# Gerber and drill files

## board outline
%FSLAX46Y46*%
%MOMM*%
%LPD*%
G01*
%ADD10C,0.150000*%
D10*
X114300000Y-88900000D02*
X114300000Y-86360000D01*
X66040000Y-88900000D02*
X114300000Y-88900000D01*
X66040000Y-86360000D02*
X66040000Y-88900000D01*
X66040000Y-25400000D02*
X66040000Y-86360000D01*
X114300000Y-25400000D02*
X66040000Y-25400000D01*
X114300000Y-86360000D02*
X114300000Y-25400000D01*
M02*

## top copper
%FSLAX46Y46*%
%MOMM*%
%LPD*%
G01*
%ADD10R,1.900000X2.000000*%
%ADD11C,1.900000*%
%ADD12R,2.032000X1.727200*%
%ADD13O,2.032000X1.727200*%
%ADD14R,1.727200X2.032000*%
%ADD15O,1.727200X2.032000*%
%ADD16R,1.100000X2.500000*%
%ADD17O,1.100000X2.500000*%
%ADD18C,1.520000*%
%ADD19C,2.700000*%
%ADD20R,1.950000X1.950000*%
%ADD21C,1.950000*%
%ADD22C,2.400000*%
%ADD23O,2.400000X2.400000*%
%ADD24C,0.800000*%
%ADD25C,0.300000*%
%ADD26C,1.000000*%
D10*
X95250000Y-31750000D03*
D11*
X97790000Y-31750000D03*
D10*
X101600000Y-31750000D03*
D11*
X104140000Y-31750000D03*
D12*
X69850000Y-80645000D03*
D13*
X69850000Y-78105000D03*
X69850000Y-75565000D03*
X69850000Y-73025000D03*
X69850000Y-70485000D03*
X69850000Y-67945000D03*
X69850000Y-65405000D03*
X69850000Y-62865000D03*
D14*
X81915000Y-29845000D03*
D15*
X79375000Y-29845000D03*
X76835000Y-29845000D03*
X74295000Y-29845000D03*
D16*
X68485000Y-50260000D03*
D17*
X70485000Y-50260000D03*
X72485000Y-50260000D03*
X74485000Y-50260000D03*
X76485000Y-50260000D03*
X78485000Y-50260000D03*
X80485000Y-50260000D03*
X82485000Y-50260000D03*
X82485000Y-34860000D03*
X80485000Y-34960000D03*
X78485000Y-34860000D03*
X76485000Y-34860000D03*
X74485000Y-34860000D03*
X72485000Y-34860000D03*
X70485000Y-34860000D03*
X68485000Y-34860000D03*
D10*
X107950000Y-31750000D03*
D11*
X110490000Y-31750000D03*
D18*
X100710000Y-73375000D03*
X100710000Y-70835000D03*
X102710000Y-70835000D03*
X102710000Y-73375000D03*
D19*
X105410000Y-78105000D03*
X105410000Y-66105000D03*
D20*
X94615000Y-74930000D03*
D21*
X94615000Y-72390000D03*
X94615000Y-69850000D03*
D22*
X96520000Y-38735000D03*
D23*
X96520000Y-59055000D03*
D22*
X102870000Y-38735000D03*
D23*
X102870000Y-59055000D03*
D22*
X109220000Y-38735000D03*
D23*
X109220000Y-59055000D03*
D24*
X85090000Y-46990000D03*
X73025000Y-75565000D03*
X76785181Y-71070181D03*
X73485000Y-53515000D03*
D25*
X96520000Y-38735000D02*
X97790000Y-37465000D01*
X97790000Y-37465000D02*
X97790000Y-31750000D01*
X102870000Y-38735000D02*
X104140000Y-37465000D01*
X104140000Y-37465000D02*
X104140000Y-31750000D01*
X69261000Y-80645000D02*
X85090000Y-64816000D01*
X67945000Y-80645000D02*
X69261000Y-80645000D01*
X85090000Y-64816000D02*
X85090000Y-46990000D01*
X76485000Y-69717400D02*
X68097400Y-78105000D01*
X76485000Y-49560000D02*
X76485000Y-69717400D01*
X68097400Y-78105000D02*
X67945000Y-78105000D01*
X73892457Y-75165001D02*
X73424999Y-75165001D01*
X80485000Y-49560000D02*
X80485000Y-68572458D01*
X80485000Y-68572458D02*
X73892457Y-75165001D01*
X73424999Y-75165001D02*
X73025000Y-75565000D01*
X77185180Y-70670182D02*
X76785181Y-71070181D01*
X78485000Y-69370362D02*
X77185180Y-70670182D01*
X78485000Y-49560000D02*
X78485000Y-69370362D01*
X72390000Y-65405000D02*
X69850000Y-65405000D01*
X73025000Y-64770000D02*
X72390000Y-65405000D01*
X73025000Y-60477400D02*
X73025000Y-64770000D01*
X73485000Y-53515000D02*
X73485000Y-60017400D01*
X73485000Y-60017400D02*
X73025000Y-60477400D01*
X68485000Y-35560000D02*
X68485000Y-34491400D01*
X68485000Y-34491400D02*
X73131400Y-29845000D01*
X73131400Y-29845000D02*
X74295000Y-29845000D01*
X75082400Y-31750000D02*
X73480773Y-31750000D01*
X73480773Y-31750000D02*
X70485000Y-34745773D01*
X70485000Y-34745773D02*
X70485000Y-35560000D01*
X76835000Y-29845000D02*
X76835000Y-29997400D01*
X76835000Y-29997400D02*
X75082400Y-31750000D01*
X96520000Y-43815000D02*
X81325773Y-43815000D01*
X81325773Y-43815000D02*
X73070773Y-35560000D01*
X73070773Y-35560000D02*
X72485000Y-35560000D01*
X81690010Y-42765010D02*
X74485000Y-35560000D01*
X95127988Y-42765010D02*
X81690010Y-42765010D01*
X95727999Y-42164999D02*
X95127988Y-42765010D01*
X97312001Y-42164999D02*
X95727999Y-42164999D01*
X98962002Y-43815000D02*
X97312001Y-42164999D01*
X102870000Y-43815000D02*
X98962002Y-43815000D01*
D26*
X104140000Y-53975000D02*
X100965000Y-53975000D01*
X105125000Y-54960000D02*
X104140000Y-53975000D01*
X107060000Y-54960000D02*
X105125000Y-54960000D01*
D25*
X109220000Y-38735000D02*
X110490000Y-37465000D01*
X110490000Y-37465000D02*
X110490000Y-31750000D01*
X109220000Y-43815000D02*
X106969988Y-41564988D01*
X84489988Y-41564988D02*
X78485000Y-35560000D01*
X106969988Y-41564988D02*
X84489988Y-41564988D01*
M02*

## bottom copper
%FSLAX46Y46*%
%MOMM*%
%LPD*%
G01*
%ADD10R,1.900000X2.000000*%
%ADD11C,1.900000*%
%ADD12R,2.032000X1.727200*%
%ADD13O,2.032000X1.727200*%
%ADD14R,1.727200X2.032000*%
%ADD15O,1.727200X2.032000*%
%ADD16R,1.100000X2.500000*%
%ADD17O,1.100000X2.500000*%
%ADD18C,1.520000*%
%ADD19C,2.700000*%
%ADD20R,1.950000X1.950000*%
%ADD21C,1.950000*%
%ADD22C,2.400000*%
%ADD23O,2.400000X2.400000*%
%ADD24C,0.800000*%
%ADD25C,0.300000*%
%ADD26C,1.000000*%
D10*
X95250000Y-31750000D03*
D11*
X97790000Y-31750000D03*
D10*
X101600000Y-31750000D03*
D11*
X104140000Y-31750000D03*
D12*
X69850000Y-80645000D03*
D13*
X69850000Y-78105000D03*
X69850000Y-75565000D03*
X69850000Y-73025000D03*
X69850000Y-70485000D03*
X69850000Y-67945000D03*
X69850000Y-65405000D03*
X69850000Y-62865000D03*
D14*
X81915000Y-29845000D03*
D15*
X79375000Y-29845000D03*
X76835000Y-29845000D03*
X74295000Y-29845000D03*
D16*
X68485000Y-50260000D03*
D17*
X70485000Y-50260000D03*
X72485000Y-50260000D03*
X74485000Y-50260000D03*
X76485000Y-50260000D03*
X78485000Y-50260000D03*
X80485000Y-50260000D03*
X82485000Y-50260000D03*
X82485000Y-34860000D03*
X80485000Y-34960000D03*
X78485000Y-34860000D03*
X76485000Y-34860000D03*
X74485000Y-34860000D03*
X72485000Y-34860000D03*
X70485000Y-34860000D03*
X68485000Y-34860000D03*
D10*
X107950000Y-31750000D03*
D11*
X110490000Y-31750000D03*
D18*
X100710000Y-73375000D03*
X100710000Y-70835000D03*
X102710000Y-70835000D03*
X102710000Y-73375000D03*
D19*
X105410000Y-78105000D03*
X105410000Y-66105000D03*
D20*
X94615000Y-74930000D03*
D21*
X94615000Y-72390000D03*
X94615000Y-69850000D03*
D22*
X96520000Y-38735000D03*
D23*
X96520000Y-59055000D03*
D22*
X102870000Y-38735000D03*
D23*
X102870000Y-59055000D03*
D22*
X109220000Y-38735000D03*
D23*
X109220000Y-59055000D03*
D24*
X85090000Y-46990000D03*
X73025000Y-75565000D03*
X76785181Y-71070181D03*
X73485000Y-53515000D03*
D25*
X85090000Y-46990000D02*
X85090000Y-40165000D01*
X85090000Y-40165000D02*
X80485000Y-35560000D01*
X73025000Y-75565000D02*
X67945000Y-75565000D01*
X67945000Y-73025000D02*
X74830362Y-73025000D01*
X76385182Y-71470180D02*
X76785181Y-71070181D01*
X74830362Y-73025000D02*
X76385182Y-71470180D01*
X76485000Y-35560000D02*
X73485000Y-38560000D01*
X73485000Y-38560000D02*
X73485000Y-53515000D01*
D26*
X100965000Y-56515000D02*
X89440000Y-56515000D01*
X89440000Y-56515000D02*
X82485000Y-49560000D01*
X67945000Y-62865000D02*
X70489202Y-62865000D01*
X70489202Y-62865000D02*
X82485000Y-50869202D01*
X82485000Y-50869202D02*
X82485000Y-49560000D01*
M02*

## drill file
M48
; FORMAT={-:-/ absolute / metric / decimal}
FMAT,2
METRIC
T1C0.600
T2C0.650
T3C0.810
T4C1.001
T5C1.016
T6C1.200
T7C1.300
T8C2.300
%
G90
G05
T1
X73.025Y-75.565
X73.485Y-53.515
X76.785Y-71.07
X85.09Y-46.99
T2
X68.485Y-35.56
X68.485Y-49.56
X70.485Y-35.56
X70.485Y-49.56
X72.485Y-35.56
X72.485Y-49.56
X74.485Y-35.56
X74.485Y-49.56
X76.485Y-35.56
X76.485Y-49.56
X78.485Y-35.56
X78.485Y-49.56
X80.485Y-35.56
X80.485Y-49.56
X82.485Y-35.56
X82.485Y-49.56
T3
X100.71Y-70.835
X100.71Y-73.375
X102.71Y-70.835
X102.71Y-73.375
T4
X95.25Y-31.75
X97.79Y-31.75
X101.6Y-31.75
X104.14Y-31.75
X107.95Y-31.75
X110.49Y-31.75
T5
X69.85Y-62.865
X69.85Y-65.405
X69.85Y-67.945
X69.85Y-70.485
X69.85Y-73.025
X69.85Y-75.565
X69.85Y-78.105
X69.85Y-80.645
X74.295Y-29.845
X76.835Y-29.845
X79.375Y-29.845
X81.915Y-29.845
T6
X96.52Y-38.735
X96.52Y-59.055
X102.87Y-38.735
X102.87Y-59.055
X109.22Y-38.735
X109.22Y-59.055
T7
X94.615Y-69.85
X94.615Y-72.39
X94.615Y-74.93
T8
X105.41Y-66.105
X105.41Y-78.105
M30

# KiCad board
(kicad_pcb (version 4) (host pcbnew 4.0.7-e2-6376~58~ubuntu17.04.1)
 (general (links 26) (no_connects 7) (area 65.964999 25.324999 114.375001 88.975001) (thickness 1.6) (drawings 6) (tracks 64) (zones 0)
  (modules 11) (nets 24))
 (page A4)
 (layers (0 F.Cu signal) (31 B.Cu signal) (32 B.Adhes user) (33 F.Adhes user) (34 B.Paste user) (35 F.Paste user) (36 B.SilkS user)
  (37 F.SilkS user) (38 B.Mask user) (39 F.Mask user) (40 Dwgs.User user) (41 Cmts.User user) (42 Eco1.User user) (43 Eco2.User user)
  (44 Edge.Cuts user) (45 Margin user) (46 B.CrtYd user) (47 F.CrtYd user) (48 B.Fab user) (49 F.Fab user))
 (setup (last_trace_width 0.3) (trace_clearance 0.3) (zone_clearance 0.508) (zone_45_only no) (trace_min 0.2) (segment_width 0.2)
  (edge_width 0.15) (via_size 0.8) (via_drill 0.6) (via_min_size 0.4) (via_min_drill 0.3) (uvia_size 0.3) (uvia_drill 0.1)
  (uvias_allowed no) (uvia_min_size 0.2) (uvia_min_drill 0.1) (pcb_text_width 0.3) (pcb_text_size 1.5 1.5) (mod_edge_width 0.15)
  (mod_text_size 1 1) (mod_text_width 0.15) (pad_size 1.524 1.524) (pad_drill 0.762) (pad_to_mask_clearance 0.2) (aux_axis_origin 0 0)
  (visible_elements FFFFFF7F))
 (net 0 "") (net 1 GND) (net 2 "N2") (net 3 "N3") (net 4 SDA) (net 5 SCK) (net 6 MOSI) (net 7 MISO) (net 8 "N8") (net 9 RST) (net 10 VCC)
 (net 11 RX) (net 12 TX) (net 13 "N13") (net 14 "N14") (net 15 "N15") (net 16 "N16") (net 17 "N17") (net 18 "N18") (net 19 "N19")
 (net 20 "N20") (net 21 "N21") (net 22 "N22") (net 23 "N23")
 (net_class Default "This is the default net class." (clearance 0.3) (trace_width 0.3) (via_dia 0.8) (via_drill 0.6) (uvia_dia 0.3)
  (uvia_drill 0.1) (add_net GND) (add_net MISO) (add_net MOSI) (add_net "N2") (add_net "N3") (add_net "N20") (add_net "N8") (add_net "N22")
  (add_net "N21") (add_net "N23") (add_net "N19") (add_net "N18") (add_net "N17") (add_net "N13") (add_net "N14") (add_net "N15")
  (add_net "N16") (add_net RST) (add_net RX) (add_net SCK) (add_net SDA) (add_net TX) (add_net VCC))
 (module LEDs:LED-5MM (layer F.Cu) (at 95.25 31.75)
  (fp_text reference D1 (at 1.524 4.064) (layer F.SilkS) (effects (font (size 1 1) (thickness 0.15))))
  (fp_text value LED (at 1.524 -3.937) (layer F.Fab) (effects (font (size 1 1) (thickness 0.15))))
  (pad 1 thru_hole rect (at 0 0 90) (size 2 1.9) (drill 1.00076) (layers *.Cu *.Mask) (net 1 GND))
  (pad 2 thru_hole circle (at 2.54 0) (size 1.9 1.9) (drill 1.00076) (layers *.Cu *.Mask) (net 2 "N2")))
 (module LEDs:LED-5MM (layer F.Cu) (at 101.6 31.75)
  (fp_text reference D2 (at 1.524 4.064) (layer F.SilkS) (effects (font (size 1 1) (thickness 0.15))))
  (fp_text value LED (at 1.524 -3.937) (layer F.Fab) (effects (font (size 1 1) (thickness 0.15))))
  (pad 1 thru_hole rect (at 0 0 90) (size 2 1.9) (drill 1.00076) (layers *.Cu *.Mask) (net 1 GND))
  (pad 2 thru_hole circle (at 2.54 0) (size 1.9 1.9) (drill 1.00076) (layers *.Cu *.Mask) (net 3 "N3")))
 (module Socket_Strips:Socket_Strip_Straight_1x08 (layer F.Cu) (at 69.85 80.645 90)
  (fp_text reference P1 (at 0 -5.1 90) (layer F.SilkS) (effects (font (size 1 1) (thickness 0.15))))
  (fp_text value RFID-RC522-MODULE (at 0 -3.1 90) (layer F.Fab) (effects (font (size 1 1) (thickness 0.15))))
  (pad 1 thru_hole rect (at 0 0 90) (size 1.7272 2.032) (drill 1.016) (layers *.Cu *.Mask) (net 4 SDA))
  (pad 2 thru_hole oval (at 2.54 0 90) (size 1.7272 2.032) (drill 1.016) (layers *.Cu *.Mask) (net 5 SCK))
  (pad 3 thru_hole oval (at 5.08 0 90) (size 1.7272 2.032) (drill 1.016) (layers *.Cu *.Mask) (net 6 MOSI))
  (pad 4 thru_hole oval (at 7.62 0 90) (size 1.7272 2.032) (drill 1.016) (layers *.Cu *.Mask) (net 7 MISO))
  (pad 5 thru_hole oval (at 10.16 0 90) (size 1.7272 2.032) (drill 1.016) (layers *.Cu *.Mask) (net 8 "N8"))
  (pad 6 thru_hole oval (at 12.7 0 90) (size 1.7272 2.032) (drill 1.016) (layers *.Cu *.Mask) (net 1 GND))
  (pad 7 thru_hole oval (at 15.24 0 90) (size 1.7272 2.032) (drill 1.016) (layers *.Cu *.Mask) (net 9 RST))
  (pad 8 thru_hole oval (at 17.78 0 90) (size 1.7272 2.032) (drill 1.016) (layers *.Cu *.Mask) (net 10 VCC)))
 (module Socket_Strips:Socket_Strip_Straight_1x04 (layer F.Cu) (at 81.915 29.845 180)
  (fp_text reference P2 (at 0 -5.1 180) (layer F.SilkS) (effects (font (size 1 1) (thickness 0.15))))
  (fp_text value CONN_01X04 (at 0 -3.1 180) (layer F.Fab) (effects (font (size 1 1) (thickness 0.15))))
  (pad 1 thru_hole rect (at 0 0 180) (size 1.7272 2.032) (drill 1.016) (layers *.Cu *.Mask) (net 10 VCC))
  (pad 2 thru_hole oval (at 2.54 0 180) (size 1.7272 2.032) (drill 1.016) (layers *.Cu *.Mask) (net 1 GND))
  (pad 3 thru_hole oval (at 5.08 0 180) (size 1.7272 2.032) (drill 1.016) (layers *.Cu *.Mask) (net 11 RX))
  (pad 4 thru_hole oval (at 7.62 0 180) (size 1.7272 2.032) (drill 1.016) (layers *.Cu *.Mask) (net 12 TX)))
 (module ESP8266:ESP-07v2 (layer F.Cu) (at 68.485 49.56 90)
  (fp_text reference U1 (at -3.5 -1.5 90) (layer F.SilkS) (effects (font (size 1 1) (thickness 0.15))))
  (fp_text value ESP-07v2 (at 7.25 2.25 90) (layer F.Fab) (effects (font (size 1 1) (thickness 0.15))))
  (pad 1 thru_hole rect (at 0 0 90) (size 2.5 1.1) (drill 0.65 (offset -0.7 0)) (layers *.Cu *.Mask F.Paste F.SilkS) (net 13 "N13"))
  (pad 2 thru_hole oval (at 0 2 90) (size 2.5 1.1) (drill 0.65 (offset -0.7 0)) (layers *.Cu *.Mask F.Paste F.SilkS) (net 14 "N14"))
  (pad 3 thru_hole oval (at 0 4 90) (size 2.5 1.1) (drill 0.65 (offset -0.7 0)) (layers *.Cu *.Mask F.Paste F.SilkS) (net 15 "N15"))
  (pad 4 thru_hole oval (at 0 6 90) (size 2.5 1.1) (drill 0.65 (offset -0.7 0)) (layers *.Cu *.Mask F.Paste F.SilkS) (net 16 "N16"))
  (pad 5 thru_hole oval (at 0 8 90) (size 2.5 1.1) (drill 0.65 (offset -0.7 0)) (layers *.Cu *.Mask F.Paste F.SilkS) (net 5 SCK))
  (pad 6 thru_hole oval (at 0 10 90) (size 2.5 1.1) (drill 0.65 (offset -0.7 0)) (layers *.Cu *.Mask F.Paste F.SilkS) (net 7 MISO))
  (pad 7 thru_hole oval (at 0 12 90) (size 2.5 1.1) (drill 0.65 (offset -0.7 0)) (layers *.Cu *.Mask F.Paste F.SilkS) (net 6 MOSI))
  (pad 8 thru_hole oval (at 0 14 90) (size 2.5 1.1) (drill 0.65 (offset -0.7 0)) (layers *.Cu *.Mask F.Paste F.SilkS) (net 10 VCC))
  (pad 9 thru_hole oval (at 14 14 90) (size 2.5 1.1) (drill 0.65 (offset 0.7 0)) (layers *.Cu *.Mask F.Paste F.SilkS) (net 1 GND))
  (pad 10 thru_hole oval (at 14 12 90) (size 2.5 1.1) (drill 0.65 (offset 0.6 0)) (layers *.Cu *.Mask F.Paste F.SilkS) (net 4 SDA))
  (pad 11 thru_hole oval (at 14 10 90) (size 2.5 1.1) (drill 0.65 (offset 0.7 0)) (layers *.Cu *.Mask F.Paste F.SilkS) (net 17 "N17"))
  (pad 12 thru_hole oval (at 14 8 90) (size 2.5 1.1) (drill 0.65 (offset 0.7 0)) (layers *.Cu *.Mask F.Paste F.SilkS) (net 9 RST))
  (pad 13 thru_hole oval (at 14 6 90) (size 2.5 1.1) (drill 0.65 (offset 0.7 0)) (layers *.Cu *.Mask F.Paste F.SilkS) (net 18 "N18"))
  (pad 14 thru_hole oval (at 14 4 90) (size 2.5 1.1) (drill 0.65 (offset 0.7 0)) (layers *.Cu *.Mask F.Paste F.SilkS) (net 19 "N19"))
  (pad 15 thru_hole oval (at 14 2 90) (size 2.5 1.1) (drill 0.65 (offset 0.7 0)) (layers *.Cu *.Mask F.Paste F.SilkS) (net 11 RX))
  (pad 16 thru_hole oval (at 14 0 90) (size 2.5 1.1) (drill 0.65 (offset 0.7 0)) (layers *.Cu *.Mask F.Paste F.SilkS) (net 12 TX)))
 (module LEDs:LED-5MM (layer F.Cu) (at 107.95 31.75)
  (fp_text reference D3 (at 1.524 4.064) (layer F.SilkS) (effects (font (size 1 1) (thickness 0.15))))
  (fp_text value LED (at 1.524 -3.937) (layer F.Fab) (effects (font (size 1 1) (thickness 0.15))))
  (pad 1 thru_hole rect (at 0 0 90) (size 2 1.9) (drill 1.00076) (layers *.Cu *.Mask) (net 1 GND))
  (pad 2 thru_hole circle (at 2.54 0) (size 1.9 1.9) (drill 1.00076) (layers *.Cu *.Mask) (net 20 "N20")))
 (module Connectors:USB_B (layer F.Cu) (at 100.71 70.835)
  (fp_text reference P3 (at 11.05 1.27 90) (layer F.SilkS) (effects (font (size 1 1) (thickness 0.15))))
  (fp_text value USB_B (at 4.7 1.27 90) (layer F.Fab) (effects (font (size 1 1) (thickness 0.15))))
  (pad 2 thru_hole circle (at 0 2.54 270) (size 1.52 1.52) (drill 0.81) (layers *.Cu *.Mask) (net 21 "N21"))
  (pad 1 thru_hole circle (at 0 0 270) (size 1.52 1.52) (drill 0.81) (layers *.Cu *.Mask) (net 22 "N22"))
  (pad 4 thru_hole circle (at 2 0 270) (size 1.52 1.52) (drill 0.81) (layers *.Cu *.Mask) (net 1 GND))
  (pad 3 thru_hole circle (at 2 2.54 270) (size 1.52 1.52) (drill 0.81) (layers *.Cu *.Mask) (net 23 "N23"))
  (pad 5 thru_hole circle (at 4.7 7.27 270) (size 2.7 2.7) (drill 2.3) (layers *.Cu *.Mask) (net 1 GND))
  (pad 5 thru_hole circle (at 4.7 -4.73 270) (size 2.7 2.7) (drill 2.3) (layers *.Cu *.Mask) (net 1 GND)))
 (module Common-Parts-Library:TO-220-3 (layer F.Cu) (at 94.615 72.39 90) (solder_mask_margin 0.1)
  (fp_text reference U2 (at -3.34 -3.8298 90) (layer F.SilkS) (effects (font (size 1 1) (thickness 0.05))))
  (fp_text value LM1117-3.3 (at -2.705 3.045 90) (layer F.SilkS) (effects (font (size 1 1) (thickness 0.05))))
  (pad 1 thru_hole rect (at -2.54 0 180) (size 1.95 1.95) (drill 1.3) (layers *.Cu *.Mask F.SilkS) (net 1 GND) (solder_mask_margin 0.2))
  (pad 2 thru_hole circle (at 0 0 180) (size 1.95 1.95) (drill 1.3) (layers *.Cu *.Mask F.SilkS) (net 10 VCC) (solder_mask_margin 0.2))
  (pad 3 thru_hole circle (at 2.54 0 180) (size 1.95 1.95) (drill 1.3) (layers *.Cu *.Mask F.SilkS) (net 22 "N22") (solder_mask_margin 0.2)))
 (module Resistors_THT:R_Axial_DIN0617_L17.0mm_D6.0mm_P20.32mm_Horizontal (layer F.Cu) (at 96.52 38.735 270)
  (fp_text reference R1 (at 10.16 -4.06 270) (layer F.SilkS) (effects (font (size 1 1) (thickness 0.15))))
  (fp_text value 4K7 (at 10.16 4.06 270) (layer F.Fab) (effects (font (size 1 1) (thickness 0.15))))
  (pad 1 thru_hole circle (at 0 0 270) (size 2.4 2.4) (drill 1.2) (layers *.Cu *.Mask) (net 2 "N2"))
  (pad 2 thru_hole oval (at 20.32 0 270) (size 2.4 2.4) (drill 1.2) (layers *.Cu *.Mask) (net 19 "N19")))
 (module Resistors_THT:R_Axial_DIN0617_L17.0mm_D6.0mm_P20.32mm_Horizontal (layer F.Cu) (at 102.87 38.735 270)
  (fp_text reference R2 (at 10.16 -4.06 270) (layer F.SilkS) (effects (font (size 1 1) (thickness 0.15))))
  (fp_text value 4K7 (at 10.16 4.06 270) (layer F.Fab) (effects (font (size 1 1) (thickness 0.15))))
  (pad 1 thru_hole circle (at 0 0 270) (size 2.4 2.4) (drill 1.2) (layers *.Cu *.Mask) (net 3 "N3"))
  (pad 2 thru_hole oval (at 20.32 0 270) (size 2.4 2.4) (drill 1.2) (layers *.Cu *.Mask) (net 18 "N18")))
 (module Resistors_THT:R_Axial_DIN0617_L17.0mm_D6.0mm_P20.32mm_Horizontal (layer F.Cu) (at 109.22 38.735 270)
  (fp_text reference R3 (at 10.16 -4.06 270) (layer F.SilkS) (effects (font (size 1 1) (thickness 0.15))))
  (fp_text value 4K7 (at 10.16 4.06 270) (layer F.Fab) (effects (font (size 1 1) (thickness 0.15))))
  (pad 1 thru_hole circle (at 0 0 270) (size 2.4 2.4) (drill 1.2) (layers *.Cu *.Mask) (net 20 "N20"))
  (pad 2 thru_hole oval (at 20.32 0 270) (size 2.4 2.4) (drill 1.2) (layers *.Cu *.Mask) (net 17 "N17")))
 (gr_line (start 114.3 88.9) (end 114.3 86.36) (layer Edge.Cuts) (width 0.15))
 (gr_line (start 66.04 88.9) (end 114.3 88.9) (layer Edge.Cuts) (width 0.15))
 (gr_line (start 66.04 86.36) (end 66.04 88.9) (layer Edge.Cuts) (width 0.15))
 (gr_line (start 66.04 25.4) (end 66.04 86.36) (layer Edge.Cuts) (width 0.15))
 (gr_line (start 114.3 25.4) (end 66.04 25.4) (layer Edge.Cuts) (width 0.15))
 (gr_line (start 114.3 86.36) (end 114.3 25.4) (layer Edge.Cuts) (width 0.15))
 (segment (start 96.52 38.735) (end 97.79 37.465) (width 0.3) (layer F.Cu) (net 2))
 (segment (start 97.79 37.465) (end 97.79 31.75) (width 0.3) (layer F.Cu) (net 2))
 (segment (start 102.87 38.735) (end 104.14 37.465) (width 0.3) (layer F.Cu) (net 3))
 (segment (start 104.14 37.465) (end 104.14 31.75) (width 0.3) (layer F.Cu) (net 3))
 (segment (start 85.09 46.99) (end 85.09 40.165) (width 0.3) (layer B.Cu) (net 4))
 (segment (start 85.09 40.165) (end 80.485 35.56) (width 0.3) (layer B.Cu) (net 4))
 (segment (start 69.261 80.645) (end 85.09 64.816) (width 0.3) (layer F.Cu) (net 4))
 (segment (start 67.945 80.645) (end 69.261 80.645) (width 0.3) (layer F.Cu) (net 4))
 (segment (start 85.09 64.816) (end 85.09 46.99) (width 0.3) (layer F.Cu) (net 4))
 (via (at 85.09 46.99) (size 0.8) (drill 0.6) (layers F.Cu B.Cu) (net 4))
 (segment (start 76.485 69.7174) (end 68.0974 78.105) (width 0.3) (layer F.Cu) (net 5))
 (segment (start 76.485 49.56) (end 76.485 69.7174) (width 0.3) (layer F.Cu) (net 5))
 (segment (start 68.0974 78.105) (end 67.945 78.105) (width 0.3) (layer F.Cu) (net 5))
 (segment (start 73.892457 75.165001) (end 73.424999 75.165001) (width 0.3) (layer F.Cu) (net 6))
 (segment (start 80.485 49.56) (end 80.485 68.572458) (width 0.3) (layer F.Cu) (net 6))
 (segment (start 80.485 68.572458) (end 73.892457 75.165001) (width 0.3) (layer F.Cu) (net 6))
 (segment (start 73.424999 75.165001) (end 73.025 75.565) (width 0.3) (layer F.Cu) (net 6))
 (segment (start 73.025 75.565) (end 67.945 75.565) (width 0.3) (layer B.Cu) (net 6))
 (via (at 73.025 75.565) (size 0.8) (drill 0.6) (layers F.Cu B.Cu) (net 6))
 (segment (start 67.945 73.025) (end 74.830362 73.025) (width 0.3) (layer B.Cu) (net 7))
 (segment (start 77.18518 70.670182) (end 76.785181 71.070181) (width 0.3) (layer F.Cu) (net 7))
 (segment (start 78.485 69.370362) (end 77.18518 70.670182) (width 0.3) (layer F.Cu) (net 7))
 (via (at 76.785181 71.070181) (size 0.8) (drill 0.6) (layers F.Cu B.Cu) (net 7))
 (segment (start 76.385182 71.47018) (end 76.785181 71.070181) (width 0.3) (layer B.Cu) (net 7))
 (segment (start 74.830362 73.025) (end 76.385182 71.47018) (width 0.3) (layer B.Cu) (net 7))
 (segment (start 78.485 49.56) (end 78.485 69.370362) (width 0.3) (layer F.Cu) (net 7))
 (segment (start 72.39 65.405) (end 69.85 65.405) (width 0.3) (layer F.Cu) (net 9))
 (segment (start 73.025 64.77) (end 72.39 65.405) (width 0.3) (layer F.Cu) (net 9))
 (segment (start 73.025 60.4774) (end 73.025 64.77) (width 0.3) (layer F.Cu) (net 9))
 (segment (start 73.485 53.515) (end 73.485 60.0174) (width 0.3) (layer F.Cu) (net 9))
 (segment (start 73.485 60.0174) (end 73.025 60.4774) (width 0.3) (layer F.Cu) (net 9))
 (via (at 73.485 53.515) (size 0.8) (drill 0.6) (layers F.Cu B.Cu) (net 9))
 (segment (start 76.485 35.56) (end 73.485 38.56) (width 0.3) (layer B.Cu) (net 9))
 (segment (start 73.485 38.56) (end 73.485 53.515) (width 0.3) (layer B.Cu) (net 9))
 (segment (start 100.965 56.515) (end 89.44 56.515) (width 1) (layer B.Cu) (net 10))
 (segment (start 89.44 56.515) (end 82.485 49.56) (width 1) (layer B.Cu) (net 10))
 (segment (start 67.945 62.865) (end 70.489202 62.865) (width 1) (layer B.Cu) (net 10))
 (segment (start 70.489202 62.865) (end 82.485 50.869202) (width 1) (layer B.Cu) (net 10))
 (segment (start 82.485 50.869202) (end 82.485 49.56) (width 1) (layer B.Cu) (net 10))
 (segment (start 68.485 35.56) (end 68.485 34.4914) (width 0.3) (layer F.Cu) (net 12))
 (segment (start 68.485 34.4914) (end 73.1314 29.845) (width 0.3) (layer F.Cu) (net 12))
 (segment (start 73.1314 29.845) (end 74.295 29.845) (width 0.3) (layer F.Cu) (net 12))
 (segment (start 75.0824 31.75) (end 73.480773 31.75) (width 0.3) (layer F.Cu) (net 11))
 (segment (start 73.480773 31.75) (end 70.485 34.745773) (width 0.3) (layer F.Cu) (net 11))
 (segment (start 70.485 34.745773) (end 70.485 35.56) (width 0.3) (layer F.Cu) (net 11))
 (segment (start 76.835 29.845) (end 76.835 29.9974) (width 0.3) (layer F.Cu) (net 11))
 (segment (start 76.835 29.9974) (end 75.0824 31.75) (width 0.3) (layer F.Cu) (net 11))
 (segment (start 96.52 43.815) (end 81.325773 43.815) (width 0.3) (layer F.Cu) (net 19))
 (segment (start 81.325773 43.815) (end 73.070773 35.56) (width 0.3) (layer F.Cu) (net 19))
 (segment (start 73.070773 35.56) (end 72.485 35.56) (width 0.3) (layer F.Cu) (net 19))
 (segment (start 81.69001 42.76501) (end 74.485 35.56) (width 0.3) (layer F.Cu) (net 18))
 (segment (start 95.127988 42.76501) (end 81.69001 42.76501) (width 0.3) (layer F.Cu) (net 18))
 (segment (start 95.727999 42.164999) (end 95.127988 42.76501) (width 0.3) (layer F.Cu) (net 18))
 (segment (start 97.312001 42.164999) (end 95.727999 42.164999) (width 0.3) (layer F.Cu) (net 18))
 (segment (start 98.962002 43.815) (end 97.312001 42.164999) (width 0.3) (layer F.Cu) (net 18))
 (segment (start 102.87 43.815) (end 98.962002 43.815) (width 0.3) (layer F.Cu) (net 18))
 (segment (start 104.14 53.975) (end 100.965 53.975) (width 1) (layer F.Cu) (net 22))
 (segment (start 105.125 54.96) (end 104.14 53.975) (width 1) (layer F.Cu) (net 22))
 (segment (start 107.06 54.96) (end 105.125 54.96) (width 1) (layer F.Cu) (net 22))
 (segment (start 109.22 38.735) (end 110.49 37.465) (width 0.3) (layer F.Cu) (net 20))
 (segment (start 110.49 37.465) (end 110.49 31.75) (width 0.3) (layer F.Cu) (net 20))
 (segment (start 109.22 43.815) (end 106.969988 41.564988) (width 0.3) (layer F.Cu) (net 17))
 (segment (start 84.489988 41.564988) (end 78.485 35.56) (width 0.3) (layer F.Cu) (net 17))
 (segment (start 106.969988 41.564988) (end 84.489988 41.564988) (width 0.3) (layer F.Cu) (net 17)))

